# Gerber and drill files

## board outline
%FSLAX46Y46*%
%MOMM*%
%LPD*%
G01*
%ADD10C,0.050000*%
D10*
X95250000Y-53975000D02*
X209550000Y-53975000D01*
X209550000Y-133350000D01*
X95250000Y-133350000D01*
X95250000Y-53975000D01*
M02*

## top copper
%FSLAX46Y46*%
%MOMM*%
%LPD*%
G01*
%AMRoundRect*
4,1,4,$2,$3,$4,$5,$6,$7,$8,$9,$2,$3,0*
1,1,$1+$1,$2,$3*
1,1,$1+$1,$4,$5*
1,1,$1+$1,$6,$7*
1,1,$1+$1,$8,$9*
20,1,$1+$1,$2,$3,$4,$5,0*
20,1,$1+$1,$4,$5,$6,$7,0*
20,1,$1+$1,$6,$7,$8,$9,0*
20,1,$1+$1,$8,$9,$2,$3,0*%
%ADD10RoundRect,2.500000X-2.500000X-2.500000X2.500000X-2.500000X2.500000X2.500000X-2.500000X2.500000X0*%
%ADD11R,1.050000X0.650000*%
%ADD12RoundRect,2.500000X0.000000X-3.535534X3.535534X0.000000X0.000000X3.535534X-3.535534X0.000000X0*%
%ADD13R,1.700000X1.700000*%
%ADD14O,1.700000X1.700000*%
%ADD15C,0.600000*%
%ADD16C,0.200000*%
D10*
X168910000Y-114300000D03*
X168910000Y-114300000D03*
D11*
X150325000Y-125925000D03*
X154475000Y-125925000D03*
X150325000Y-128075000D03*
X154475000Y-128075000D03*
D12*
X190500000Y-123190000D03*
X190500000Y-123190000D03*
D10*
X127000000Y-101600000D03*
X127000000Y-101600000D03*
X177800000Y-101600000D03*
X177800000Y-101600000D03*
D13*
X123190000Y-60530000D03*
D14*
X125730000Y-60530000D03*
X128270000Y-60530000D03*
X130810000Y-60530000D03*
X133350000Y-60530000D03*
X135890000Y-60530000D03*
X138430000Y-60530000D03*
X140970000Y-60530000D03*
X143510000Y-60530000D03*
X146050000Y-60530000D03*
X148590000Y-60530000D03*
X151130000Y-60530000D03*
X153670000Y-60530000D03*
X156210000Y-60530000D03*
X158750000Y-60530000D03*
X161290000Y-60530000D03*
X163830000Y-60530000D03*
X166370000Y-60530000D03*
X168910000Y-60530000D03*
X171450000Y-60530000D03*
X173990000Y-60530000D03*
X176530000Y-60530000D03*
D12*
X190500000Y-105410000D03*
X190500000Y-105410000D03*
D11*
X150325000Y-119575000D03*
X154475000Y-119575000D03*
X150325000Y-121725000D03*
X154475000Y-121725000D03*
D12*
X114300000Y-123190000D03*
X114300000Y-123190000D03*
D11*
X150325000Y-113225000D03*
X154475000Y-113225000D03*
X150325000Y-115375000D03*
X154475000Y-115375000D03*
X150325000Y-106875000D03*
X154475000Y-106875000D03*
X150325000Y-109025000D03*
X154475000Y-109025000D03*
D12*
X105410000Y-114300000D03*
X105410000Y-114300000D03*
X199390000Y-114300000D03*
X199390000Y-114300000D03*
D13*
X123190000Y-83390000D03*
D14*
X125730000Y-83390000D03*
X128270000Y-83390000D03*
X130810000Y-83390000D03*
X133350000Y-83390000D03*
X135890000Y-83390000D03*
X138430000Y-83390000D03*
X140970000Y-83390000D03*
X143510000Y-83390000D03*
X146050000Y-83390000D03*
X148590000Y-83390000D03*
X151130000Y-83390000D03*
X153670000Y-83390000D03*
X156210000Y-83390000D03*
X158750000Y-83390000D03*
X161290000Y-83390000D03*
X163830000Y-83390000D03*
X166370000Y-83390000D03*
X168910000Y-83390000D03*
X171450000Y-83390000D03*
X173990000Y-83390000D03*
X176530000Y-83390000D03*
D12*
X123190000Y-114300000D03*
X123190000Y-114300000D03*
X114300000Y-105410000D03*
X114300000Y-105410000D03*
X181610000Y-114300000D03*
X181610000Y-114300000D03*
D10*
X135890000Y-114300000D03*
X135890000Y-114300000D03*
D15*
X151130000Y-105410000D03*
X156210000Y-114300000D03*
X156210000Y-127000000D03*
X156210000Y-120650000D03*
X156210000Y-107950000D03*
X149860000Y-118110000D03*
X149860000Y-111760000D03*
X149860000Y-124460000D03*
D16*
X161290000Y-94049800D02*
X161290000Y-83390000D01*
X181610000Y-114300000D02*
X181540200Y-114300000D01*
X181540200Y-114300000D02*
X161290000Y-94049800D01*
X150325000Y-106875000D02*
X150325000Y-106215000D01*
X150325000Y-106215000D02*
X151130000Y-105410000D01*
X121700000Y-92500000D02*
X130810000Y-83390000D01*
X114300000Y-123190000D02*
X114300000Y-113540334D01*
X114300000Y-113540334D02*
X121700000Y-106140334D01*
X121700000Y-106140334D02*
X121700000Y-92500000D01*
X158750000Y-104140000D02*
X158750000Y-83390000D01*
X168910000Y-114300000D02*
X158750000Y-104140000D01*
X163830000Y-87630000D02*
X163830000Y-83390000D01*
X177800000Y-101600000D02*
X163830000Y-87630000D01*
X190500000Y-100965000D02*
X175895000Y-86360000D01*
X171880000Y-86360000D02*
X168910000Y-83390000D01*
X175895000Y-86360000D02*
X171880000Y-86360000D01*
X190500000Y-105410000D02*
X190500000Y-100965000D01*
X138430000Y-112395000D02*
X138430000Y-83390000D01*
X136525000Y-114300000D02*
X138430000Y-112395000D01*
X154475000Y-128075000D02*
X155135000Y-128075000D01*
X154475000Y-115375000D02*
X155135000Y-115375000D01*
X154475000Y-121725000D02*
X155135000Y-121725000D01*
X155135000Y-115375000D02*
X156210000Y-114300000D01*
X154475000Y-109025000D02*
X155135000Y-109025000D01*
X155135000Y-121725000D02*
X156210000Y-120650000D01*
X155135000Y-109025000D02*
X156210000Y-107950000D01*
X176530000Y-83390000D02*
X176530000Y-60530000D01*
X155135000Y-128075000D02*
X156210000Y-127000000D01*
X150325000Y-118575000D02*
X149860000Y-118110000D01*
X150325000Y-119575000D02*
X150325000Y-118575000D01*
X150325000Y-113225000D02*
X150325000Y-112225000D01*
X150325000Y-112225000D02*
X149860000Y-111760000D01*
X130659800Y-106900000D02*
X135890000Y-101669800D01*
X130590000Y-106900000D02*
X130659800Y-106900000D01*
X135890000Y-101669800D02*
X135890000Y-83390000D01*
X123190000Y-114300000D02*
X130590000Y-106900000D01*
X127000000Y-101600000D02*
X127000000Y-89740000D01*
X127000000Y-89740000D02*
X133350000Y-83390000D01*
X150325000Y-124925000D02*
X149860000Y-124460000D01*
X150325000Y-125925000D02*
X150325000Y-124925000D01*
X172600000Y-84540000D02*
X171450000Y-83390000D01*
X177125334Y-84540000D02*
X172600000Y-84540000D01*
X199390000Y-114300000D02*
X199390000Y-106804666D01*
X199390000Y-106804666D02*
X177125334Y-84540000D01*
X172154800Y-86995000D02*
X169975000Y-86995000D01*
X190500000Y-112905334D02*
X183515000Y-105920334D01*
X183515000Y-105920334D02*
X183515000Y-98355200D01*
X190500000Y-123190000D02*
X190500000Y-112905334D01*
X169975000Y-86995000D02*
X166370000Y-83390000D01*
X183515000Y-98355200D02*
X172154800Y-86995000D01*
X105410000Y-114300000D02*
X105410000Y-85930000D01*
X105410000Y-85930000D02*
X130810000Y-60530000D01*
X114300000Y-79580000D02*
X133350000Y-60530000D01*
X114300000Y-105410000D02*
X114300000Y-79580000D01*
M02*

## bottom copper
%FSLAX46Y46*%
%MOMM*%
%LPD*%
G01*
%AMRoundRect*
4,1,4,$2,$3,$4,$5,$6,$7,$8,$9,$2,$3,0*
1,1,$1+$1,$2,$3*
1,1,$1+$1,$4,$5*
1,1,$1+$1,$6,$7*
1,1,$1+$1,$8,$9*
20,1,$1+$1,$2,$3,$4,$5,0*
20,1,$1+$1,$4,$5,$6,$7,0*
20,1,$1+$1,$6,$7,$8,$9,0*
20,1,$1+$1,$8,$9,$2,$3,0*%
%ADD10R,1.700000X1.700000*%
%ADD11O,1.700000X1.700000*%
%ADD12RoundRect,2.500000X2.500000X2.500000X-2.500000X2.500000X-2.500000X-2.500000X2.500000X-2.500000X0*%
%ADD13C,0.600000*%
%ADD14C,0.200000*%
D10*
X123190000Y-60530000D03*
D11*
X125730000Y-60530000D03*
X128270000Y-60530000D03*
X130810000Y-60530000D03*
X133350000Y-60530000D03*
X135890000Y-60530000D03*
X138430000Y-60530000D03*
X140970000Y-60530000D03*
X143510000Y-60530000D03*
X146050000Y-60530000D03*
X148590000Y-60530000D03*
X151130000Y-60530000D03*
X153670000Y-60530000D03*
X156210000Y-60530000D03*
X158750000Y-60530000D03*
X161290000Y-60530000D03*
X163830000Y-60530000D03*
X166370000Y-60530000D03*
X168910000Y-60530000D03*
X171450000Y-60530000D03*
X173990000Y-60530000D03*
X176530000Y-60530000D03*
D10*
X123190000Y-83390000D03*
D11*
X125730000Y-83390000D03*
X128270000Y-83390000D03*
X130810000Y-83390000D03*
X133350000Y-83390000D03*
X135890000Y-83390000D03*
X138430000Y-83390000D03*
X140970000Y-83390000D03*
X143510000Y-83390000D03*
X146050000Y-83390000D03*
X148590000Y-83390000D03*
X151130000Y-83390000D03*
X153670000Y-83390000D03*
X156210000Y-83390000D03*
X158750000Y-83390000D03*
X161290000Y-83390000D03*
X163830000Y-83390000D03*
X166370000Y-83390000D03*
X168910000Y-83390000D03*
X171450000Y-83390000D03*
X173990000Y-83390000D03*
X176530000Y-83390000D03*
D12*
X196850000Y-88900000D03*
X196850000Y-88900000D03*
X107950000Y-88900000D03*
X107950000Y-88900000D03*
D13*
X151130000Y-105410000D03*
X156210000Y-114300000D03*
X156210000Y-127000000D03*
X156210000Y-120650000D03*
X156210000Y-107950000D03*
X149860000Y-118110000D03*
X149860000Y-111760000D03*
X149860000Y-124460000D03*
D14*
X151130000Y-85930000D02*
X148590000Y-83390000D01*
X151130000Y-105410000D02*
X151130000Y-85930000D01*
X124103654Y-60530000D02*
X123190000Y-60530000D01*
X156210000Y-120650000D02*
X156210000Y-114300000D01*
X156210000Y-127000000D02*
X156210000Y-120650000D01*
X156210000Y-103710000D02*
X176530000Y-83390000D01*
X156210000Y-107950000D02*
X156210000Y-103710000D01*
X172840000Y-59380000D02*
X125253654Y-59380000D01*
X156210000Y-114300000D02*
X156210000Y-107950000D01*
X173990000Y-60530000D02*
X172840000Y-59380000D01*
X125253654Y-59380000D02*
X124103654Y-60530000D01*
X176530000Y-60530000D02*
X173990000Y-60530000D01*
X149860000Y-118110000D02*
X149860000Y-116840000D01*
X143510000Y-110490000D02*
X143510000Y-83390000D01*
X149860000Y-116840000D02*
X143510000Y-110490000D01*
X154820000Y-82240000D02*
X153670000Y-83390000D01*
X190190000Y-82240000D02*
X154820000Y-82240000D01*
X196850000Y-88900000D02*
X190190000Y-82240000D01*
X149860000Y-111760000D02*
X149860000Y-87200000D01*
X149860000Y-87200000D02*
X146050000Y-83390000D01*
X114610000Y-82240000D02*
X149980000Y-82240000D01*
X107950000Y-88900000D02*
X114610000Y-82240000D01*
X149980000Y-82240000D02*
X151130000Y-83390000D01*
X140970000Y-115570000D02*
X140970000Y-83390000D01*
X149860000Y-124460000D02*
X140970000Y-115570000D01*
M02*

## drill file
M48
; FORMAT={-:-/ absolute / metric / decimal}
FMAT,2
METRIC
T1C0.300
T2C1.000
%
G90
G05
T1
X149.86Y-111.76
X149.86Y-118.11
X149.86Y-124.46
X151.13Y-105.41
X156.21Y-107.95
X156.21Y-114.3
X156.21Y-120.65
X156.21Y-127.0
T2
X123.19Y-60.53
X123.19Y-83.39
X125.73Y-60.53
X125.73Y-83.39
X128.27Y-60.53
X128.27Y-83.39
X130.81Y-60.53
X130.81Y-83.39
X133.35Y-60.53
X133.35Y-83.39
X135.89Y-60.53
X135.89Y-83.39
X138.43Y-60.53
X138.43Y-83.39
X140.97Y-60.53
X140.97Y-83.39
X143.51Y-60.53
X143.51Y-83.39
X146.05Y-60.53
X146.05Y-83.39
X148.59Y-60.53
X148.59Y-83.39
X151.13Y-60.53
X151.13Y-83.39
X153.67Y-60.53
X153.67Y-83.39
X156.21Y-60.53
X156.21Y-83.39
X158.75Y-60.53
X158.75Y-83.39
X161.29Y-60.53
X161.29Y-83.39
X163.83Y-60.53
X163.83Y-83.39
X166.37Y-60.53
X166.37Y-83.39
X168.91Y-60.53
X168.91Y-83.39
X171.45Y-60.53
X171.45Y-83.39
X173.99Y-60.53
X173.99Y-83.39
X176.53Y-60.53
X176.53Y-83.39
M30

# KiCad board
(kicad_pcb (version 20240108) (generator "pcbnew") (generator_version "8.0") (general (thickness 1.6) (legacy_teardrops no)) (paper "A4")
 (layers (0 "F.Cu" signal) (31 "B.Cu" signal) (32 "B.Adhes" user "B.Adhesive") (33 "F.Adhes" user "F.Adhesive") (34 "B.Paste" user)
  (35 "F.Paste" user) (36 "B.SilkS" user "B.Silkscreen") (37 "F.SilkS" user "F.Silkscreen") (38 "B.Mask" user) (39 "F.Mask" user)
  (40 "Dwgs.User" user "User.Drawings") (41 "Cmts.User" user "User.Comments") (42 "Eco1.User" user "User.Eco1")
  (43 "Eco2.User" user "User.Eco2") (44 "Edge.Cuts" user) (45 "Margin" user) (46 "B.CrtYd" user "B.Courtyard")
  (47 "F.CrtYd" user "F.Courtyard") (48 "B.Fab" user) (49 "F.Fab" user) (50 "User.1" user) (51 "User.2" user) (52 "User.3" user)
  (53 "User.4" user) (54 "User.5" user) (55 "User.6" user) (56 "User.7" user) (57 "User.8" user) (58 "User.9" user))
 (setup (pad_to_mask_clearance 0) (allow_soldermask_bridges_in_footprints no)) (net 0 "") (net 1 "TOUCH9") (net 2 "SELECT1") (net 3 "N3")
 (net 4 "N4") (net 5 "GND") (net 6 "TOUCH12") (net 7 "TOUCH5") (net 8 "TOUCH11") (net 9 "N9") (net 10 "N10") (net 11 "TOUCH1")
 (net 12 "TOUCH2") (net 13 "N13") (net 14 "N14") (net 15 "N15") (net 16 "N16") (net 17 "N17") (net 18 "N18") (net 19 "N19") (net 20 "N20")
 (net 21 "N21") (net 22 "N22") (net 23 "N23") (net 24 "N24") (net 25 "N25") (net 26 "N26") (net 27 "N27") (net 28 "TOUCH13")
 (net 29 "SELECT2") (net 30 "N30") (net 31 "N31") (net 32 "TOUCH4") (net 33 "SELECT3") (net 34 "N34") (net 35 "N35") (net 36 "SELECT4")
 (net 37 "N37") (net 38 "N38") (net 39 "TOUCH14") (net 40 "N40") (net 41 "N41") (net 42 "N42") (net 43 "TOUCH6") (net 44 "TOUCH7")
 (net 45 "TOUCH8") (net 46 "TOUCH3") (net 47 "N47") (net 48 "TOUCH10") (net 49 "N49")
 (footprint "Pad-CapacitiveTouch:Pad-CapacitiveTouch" (layer "F.Cu") (at 168.91 114.3)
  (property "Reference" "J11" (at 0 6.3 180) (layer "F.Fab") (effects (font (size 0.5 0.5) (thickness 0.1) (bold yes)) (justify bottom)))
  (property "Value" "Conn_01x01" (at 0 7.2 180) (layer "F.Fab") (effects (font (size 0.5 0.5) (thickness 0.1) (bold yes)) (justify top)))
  (pad "1" smd roundrect (at 0 0) (size 10 10) (layers "F.Cu") (roundrect_rratio 0.25) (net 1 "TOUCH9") (thermal_bridge_angle 0))
  (pad "1" smd roundrect (at 0 0) (size 10 10) (layers "F.Cu" "F.Mask") (roundrect_rratio 0.25) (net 1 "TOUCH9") (thermal_bridge_angle 0)))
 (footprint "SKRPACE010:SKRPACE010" (layer "F.Cu") (at 152.4 127)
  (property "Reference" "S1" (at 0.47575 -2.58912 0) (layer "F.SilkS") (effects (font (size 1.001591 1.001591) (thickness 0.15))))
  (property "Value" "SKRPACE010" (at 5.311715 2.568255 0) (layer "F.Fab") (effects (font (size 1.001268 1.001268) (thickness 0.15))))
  (pad "1" smd rect (at -2.075 -1.075) (size 1.05 0.65) (layers "F.Cu" "F.Paste" "F.Mask") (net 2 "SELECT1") (solder_mask_margin 0.102))
  (pad "2" smd rect (at 2.075 -1.075) (size 1.05 0.65) (layers "F.Cu" "F.Paste" "F.Mask") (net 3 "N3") (solder_mask_margin 0.102))
  (pad "3" smd rect (at -2.075 1.075) (size 1.05 0.65) (layers "F.Cu" "F.Paste" "F.Mask") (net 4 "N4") (solder_mask_margin 0.102))
  (pad "4" smd rect (at 2.075 1.075) (size 1.05 0.65) (layers "F.Cu" "F.Paste" "F.Mask") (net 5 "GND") (solder_mask_margin 0.102)))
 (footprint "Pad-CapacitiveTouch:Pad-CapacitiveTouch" (layer "F.Cu") (at 190.5 123.19 45)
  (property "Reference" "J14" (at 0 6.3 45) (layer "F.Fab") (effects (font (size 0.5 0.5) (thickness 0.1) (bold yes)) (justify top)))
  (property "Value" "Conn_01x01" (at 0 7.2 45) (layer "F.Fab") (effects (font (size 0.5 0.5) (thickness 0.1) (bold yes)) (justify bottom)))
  (pad "1" smd roundrect (at 0 0 45) (size 10 10) (layers "F.Cu") (roundrect_rratio 0.25) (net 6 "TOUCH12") (thermal_bridge_angle 0))
  (pad "1" smd roundrect (at 0 0 45) (size 10 10) (layers "F.Cu" "F.Mask") (roundrect_rratio 0.25) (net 6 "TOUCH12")
   (thermal_bridge_angle 0)))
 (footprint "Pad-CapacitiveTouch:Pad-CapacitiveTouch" (layer "F.Cu") (at 127 101.6)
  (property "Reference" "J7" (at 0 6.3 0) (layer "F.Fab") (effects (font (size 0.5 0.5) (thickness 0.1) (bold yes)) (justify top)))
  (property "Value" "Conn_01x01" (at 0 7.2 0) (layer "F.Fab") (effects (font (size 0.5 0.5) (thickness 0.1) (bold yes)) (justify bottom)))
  (pad "1" smd roundrect (at 0 0) (size 10 10) (layers "F.Cu") (roundrect_rratio 0.25) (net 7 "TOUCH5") (thermal_bridge_angle 0))
  (pad "1" smd roundrect (at 0 0) (size 10 10) (layers "F.Cu" "F.Mask") (roundrect_rratio 0.25) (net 7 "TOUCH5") (thermal_bridge_angle 0)))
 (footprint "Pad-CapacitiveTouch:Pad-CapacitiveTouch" (layer "F.Cu") (at 177.8 101.6)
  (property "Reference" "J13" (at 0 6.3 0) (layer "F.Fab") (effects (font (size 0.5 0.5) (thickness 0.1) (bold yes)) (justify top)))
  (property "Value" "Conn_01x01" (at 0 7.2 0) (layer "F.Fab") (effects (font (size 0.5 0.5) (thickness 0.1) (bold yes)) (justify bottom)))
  (pad "1" smd roundrect (at 0 0) (size 10 10) (layers "F.Cu") (roundrect_rratio 0.25) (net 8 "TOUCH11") (thermal_bridge_angle 0))
  (pad "1" smd roundrect (at 0 0) (size 10 10) (layers "F.Cu" "F.Mask") (roundrect_rratio 0.25) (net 8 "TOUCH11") (thermal_bridge_angle 0)))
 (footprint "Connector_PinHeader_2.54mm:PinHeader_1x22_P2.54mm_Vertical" (layer "F.Cu") (at 123.19 60.53 90)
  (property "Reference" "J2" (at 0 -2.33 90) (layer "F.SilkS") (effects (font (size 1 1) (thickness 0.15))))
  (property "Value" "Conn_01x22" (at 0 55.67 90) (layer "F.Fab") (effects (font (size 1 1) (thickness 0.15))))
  (pad "1" thru_hole rect (at 0 0 90) (size 1.7 1.7) (drill 1) (layers "*.Cu" "*.Mask") (remove_unused_layers no) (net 5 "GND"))
  (pad "2" thru_hole oval (at 0 2.54 90) (size 1.7 1.7) (drill 1) (layers "*.Cu" "*.Mask") (remove_unused_layers no) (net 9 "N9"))
  (pad "3" thru_hole oval (at 0 5.08 90) (size 1.7 1.7) (drill 1) (layers "*.Cu" "*.Mask") (remove_unused_layers no) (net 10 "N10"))
  (pad "4" thru_hole oval (at 0 7.62 90) (size 1.7 1.7) (drill 1) (layers "*.Cu" "*.Mask") (remove_unused_layers no) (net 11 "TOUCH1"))
  (pad "5" thru_hole oval (at 0 10.16 90) (size 1.7 1.7) (drill 1) (layers "*.Cu" "*.Mask") (remove_unused_layers no) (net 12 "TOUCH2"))
  (pad "6" thru_hole oval (at 0 12.7 90) (size 1.7 1.7) (drill 1) (layers "*.Cu" "*.Mask") (remove_unused_layers no) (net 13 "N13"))
  (pad "7" thru_hole oval (at 0 15.24 90) (size 1.7 1.7) (drill 1) (layers "*.Cu" "*.Mask") (remove_unused_layers no) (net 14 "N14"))
  (pad "8" thru_hole oval (at 0 17.78 90) (size 1.7 1.7) (drill 1) (layers "*.Cu" "*.Mask") (remove_unused_layers no) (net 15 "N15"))
  (pad "9" thru_hole oval (at 0 20.32 90) (size 1.7 1.7) (drill 1) (layers "*.Cu" "*.Mask") (remove_unused_layers no) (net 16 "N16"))
  (pad "10" thru_hole oval (at 0 22.86 90) (size 1.7 1.7) (drill 1) (layers "*.Cu" "*.Mask") (remove_unused_layers no) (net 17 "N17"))
  (pad "11" thru_hole oval (at 0 25.4 90) (size 1.7 1.7) (drill 1) (layers "*.Cu" "*.Mask") (remove_unused_layers no) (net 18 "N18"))
  (pad "12" thru_hole oval (at 0 27.94 90) (size 1.7 1.7) (drill 1) (layers "*.Cu" "*.Mask") (remove_unused_layers no) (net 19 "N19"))
  (pad "13" thru_hole oval (at 0 30.48 90) (size 1.7 1.7) (drill 1) (layers "*.Cu" "*.Mask") (remove_unused_layers no) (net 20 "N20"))
  (pad "14" thru_hole oval (at 0 33.02 90) (size 1.7 1.7) (drill 1) (layers "*.Cu" "*.Mask") (remove_unused_layers no) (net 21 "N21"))
  (pad "15" thru_hole oval (at 0 35.56 90) (size 1.7 1.7) (drill 1) (layers "*.Cu" "*.Mask") (remove_unused_layers no) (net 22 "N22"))
  (pad "16" thru_hole oval (at 0 38.1 90) (size 1.7 1.7) (drill 1) (layers "*.Cu" "*.Mask") (remove_unused_layers no) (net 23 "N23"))
  (pad "17" thru_hole oval (at 0 40.64 90) (size 1.7 1.7) (drill 1) (layers "*.Cu" "*.Mask") (remove_unused_layers no) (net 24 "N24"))
  (pad "18" thru_hole oval (at 0 43.18 90) (size 1.7 1.7) (drill 1) (layers "*.Cu" "*.Mask") (remove_unused_layers no) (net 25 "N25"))
  (pad "19" thru_hole oval (at 0 45.72 90) (size 1.7 1.7) (drill 1) (layers "*.Cu" "*.Mask") (remove_unused_layers no) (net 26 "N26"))
  (pad "20" thru_hole oval (at 0 48.26 90) (size 1.7 1.7) (drill 1) (layers "*.Cu" "*.Mask") (remove_unused_layers no) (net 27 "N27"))
  (pad "21" thru_hole oval (at 0 50.8 90) (size 1.7 1.7) (drill 1) (layers "*.Cu" "*.Mask") (remove_unused_layers no) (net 5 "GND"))
  (pad "22" thru_hole oval (at 0 53.34 90) (size 1.7 1.7) (drill 1) (layers "*.Cu" "*.Mask") (remove_unused_layers no) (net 5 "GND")))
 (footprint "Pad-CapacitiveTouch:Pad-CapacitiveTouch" (layer "F.Cu") (at 190.5 105.41 45)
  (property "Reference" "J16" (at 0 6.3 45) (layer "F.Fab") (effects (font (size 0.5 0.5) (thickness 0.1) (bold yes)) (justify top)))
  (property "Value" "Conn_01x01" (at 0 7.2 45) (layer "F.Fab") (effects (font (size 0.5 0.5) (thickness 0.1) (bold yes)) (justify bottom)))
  (pad "1" smd roundrect (at 0 0 45) (size 10 10) (layers "F.Cu") (roundrect_rratio 0.25) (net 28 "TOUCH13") (thermal_bridge_angle 0))
  (pad "1" smd roundrect (at 0 0 45) (size 10 10) (layers "F.Cu" "F.Mask") (roundrect_rratio 0.25) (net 28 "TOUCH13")
   (thermal_bridge_angle 0)))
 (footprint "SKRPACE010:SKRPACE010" (layer "F.Cu") (at 152.4 120.65)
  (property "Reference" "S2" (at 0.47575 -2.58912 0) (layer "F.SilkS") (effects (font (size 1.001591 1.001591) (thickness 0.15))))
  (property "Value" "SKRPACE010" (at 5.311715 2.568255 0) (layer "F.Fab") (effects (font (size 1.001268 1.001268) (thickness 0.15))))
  (pad "1" smd rect (at -2.075 -1.075) (size 1.05 0.65) (layers "F.Cu" "F.Paste" "F.Mask") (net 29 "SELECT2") (solder_mask_margin 0.102))
  (pad "2" smd rect (at 2.075 -1.075) (size 1.05 0.65) (layers "F.Cu" "F.Paste" "F.Mask") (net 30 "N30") (solder_mask_margin 0.102))
  (pad "3" smd rect (at -2.075 1.075) (size 1.05 0.65) (layers "F.Cu" "F.Paste" "F.Mask") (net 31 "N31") (solder_mask_margin 0.102))
  (pad "4" smd rect (at 2.075 1.075) (size 1.05 0.65) (layers "F.Cu" "F.Paste" "F.Mask") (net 5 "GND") (solder_mask_margin 0.102)))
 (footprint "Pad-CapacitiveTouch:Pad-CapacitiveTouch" (layer "F.Cu") (at 114.3 123.19 45)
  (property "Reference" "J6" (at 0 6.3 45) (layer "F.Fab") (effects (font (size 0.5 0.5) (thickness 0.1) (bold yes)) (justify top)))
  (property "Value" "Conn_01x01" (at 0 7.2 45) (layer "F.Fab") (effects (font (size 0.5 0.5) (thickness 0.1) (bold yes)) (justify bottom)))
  (pad "1" smd roundrect (at 0 0 45) (size 10 10) (layers "F.Cu") (roundrect_rratio 0.25) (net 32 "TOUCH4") (thermal_bridge_angle 0))
  (pad "1" smd roundrect (at 0 0 45) (size 10 10) (layers "F.Cu" "F.Mask") (roundrect_rratio 0.25) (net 32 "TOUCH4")
   (thermal_bridge_angle 0)))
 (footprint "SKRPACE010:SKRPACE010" (layer "F.Cu") (at 152.4 114.3)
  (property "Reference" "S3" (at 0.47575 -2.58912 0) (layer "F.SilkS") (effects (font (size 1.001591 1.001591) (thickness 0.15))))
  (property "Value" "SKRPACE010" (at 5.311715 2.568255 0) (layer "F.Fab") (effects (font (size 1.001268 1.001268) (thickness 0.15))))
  (pad "1" smd rect (at -2.075 -1.075) (size 1.05 0.65) (layers "F.Cu" "F.Paste" "F.Mask") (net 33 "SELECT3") (solder_mask_margin 0.102))
  (pad "2" smd rect (at 2.075 -1.075) (size 1.05 0.65) (layers "F.Cu" "F.Paste" "F.Mask") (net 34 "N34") (solder_mask_margin 0.102))
  (pad "3" smd rect (at -2.075 1.075) (size 1.05 0.65) (layers "F.Cu" "F.Paste" "F.Mask") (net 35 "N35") (solder_mask_margin 0.102))
  (pad "4" smd rect (at 2.075 1.075) (size 1.05 0.65) (layers "F.Cu" "F.Paste" "F.Mask") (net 5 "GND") (solder_mask_margin 0.102)))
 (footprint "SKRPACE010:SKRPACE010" (layer "F.Cu") (at 152.4 107.95)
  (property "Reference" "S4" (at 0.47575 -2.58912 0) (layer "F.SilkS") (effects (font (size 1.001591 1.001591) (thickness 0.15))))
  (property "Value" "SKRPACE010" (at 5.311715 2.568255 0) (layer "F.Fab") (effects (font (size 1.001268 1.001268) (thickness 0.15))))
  (pad "1" smd rect (at -2.075 -1.075) (size 1.05 0.65) (layers "F.Cu" "F.Paste" "F.Mask") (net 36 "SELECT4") (solder_mask_margin 0.102))
  (pad "2" smd rect (at 2.075 -1.075) (size 1.05 0.65) (layers "F.Cu" "F.Paste" "F.Mask") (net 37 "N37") (solder_mask_margin 0.102))
  (pad "3" smd rect (at -2.075 1.075) (size 1.05 0.65) (layers "F.Cu" "F.Paste" "F.Mask") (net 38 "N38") (solder_mask_margin 0.102))
  (pad "4" smd rect (at 2.075 1.075) (size 1.05 0.65) (layers "F.Cu" "F.Paste" "F.Mask") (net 5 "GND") (solder_mask_margin 0.102)))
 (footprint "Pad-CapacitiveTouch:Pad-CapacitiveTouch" (layer "F.Cu") (at 105.41 114.3 45)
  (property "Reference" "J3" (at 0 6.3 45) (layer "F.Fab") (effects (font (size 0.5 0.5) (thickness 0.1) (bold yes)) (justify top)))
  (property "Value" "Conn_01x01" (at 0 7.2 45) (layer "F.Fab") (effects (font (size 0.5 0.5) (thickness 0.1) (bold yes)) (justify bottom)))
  (pad "1" smd roundrect (at 0 0 45) (size 10 10) (layers "F.Cu") (roundrect_rratio 0.25) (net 11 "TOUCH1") (thermal_bridge_angle 0))
  (pad "1" smd roundrect (at 0 0 45) (size 10 10) (layers "F.Cu" "F.Mask") (roundrect_rratio 0.25) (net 11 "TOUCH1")
   (thermal_bridge_angle 0)))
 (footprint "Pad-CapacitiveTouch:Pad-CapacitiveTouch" (layer "F.Cu") (at 199.39 114.3 45)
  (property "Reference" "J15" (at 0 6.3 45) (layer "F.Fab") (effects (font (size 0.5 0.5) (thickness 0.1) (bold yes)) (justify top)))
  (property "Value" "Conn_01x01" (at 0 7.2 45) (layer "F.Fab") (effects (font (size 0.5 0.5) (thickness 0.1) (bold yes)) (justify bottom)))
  (pad "1" smd roundrect (at 0 0 45) (size 10 10) (layers "F.Cu") (roundrect_rratio 0.25) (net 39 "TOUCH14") (thermal_bridge_angle 0))
  (pad "1" smd roundrect (at 0 0 45) (size 10 10) (layers "F.Cu" "F.Mask") (roundrect_rratio 0.25) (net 39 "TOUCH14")
   (thermal_bridge_angle 0)))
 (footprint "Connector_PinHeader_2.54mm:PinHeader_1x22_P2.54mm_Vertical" (layer "F.Cu") (at 123.19 83.39 90)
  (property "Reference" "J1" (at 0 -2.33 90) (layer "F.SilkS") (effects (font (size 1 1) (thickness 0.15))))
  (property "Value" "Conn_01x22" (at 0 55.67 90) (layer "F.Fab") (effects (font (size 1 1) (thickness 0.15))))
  (pad "1" thru_hole rect (at 0 0 90) (size 1.7 1.7) (drill 1) (layers "*.Cu" "*.Mask") (remove_unused_layers no) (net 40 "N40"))
  (pad "2" thru_hole oval (at 0 2.54 90) (size 1.7 1.7) (drill 1) (layers "*.Cu" "*.Mask") (remove_unused_layers no) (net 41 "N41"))
  (pad "3" thru_hole oval (at 0 5.08 90) (size 1.7 1.7) (drill 1) (layers "*.Cu" "*.Mask") (remove_unused_layers no) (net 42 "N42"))
  (pad "4" thru_hole oval (at 0 7.62 90) (size 1.7 1.7) (drill 1) (layers "*.Cu" "*.Mask") (remove_unused_layers no) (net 32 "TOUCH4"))
  (pad "5" thru_hole oval (at 0 10.16 90) (size 1.7 1.7) (drill 1) (layers "*.Cu" "*.Mask") (remove_unused_layers no) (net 7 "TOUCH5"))
  (pad "6" thru_hole oval (at 0 12.7 90) (size 1.7 1.7) (drill 1) (layers "*.Cu" "*.Mask") (remove_unused_layers no) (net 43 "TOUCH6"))
  (pad "7" thru_hole oval (at 0 15.24 90) (size 1.7 1.7) (drill 1) (layers "*.Cu" "*.Mask") (remove_unused_layers no) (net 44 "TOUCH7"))
  (pad "8" thru_hole oval (at 0 17.78 90) (size 1.7 1.7) (drill 1) (layers "*.Cu" "*.Mask") (remove_unused_layers no) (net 2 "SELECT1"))
  (pad "9" thru_hole oval (at 0 20.32 90) (size 1.7 1.7) (drill 1) (layers "*.Cu" "*.Mask") (remove_unused_layers no) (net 29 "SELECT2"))
  (pad "10" thru_hole oval (at 0 22.86 90) (size 1.7 1.7) (drill 1) (layers "*.Cu" "*.Mask") (remove_unused_layers no) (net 33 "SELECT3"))
  (pad "11" thru_hole oval (at 0 25.4 90) (size 1.7 1.7) (drill 1) (layers "*.Cu" "*.Mask") (remove_unused_layers no) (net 36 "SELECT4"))
  (pad "12" thru_hole oval (at 0 27.94 90) (size 1.7 1.7) (drill 1) (layers "*.Cu" "*.Mask") (remove_unused_layers no) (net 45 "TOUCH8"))
  (pad "13" thru_hole oval (at 0 30.48 90) (size 1.7 1.7) (drill 1) (layers "*.Cu" "*.Mask") (remove_unused_layers no) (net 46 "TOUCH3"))
  (pad "14" thru_hole oval (at 0 33.02 90) (size 1.7 1.7) (drill 1) (layers "*.Cu" "*.Mask") (remove_unused_layers no) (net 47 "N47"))
  (pad "15" thru_hole oval (at 0 35.56 90) (size 1.7 1.7) (drill 1) (layers "*.Cu" "*.Mask") (remove_unused_layers no) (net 1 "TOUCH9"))
  (pad "16" thru_hole oval (at 0 38.1 90) (size 1.7 1.7) (drill 1) (layers "*.Cu" "*.Mask") (remove_unused_layers no) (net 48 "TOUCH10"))
  (pad "17" thru_hole oval (at 0 40.64 90) (size 1.7 1.7) (drill 1) (layers "*.Cu" "*.Mask") (remove_unused_layers no) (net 8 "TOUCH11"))
  (pad "18" thru_hole oval (at 0 43.18 90) (size 1.7 1.7) (drill 1) (layers "*.Cu" "*.Mask") (remove_unused_layers no) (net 6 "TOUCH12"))
  (pad "19" thru_hole oval (at 0 45.72 90) (size 1.7 1.7) (drill 1) (layers "*.Cu" "*.Mask") (remove_unused_layers no) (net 28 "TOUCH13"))
  (pad "20" thru_hole oval (at 0 48.26 90) (size 1.7 1.7) (drill 1) (layers "*.Cu" "*.Mask") (remove_unused_layers no) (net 39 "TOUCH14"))
  (pad "21" thru_hole oval (at 0 50.8 90) (size 1.7 1.7) (drill 1) (layers "*.Cu" "*.Mask") (remove_unused_layers no) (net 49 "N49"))
  (pad "22" thru_hole oval (at 0 53.34 90) (size 1.7 1.7) (drill 1) (layers "*.Cu" "*.Mask") (remove_unused_layers no) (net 5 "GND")))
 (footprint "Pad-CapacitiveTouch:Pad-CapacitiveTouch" (layer "F.Cu") (at 123.19 114.3 45)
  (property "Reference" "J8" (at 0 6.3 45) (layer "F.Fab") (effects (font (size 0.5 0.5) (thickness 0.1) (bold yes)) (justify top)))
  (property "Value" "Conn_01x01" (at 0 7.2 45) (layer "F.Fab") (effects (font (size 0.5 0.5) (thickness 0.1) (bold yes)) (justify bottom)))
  (pad "1" smd roundrect (at 0 0 45) (size 10 10) (layers "F.Cu") (roundrect_rratio 0.25) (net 43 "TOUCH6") (thermal_bridge_angle 0))
  (pad "1" smd roundrect (at 0 0 45) (size 10 10) (layers "F.Cu" "F.Mask") (roundrect_rratio 0.25) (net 43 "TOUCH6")
   (thermal_bridge_angle 0)))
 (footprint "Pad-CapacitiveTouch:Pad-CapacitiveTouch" (layer "F.Cu") (at 114.3 105.41 45)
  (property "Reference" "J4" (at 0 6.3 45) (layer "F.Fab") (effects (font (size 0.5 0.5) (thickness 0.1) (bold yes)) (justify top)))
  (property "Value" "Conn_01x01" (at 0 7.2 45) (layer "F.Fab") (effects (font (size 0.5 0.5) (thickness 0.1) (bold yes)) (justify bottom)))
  (pad "1" smd roundrect (at 0 0 45) (size 10 10) (layers "F.Cu") (roundrect_rratio 0.25) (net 12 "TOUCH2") (thermal_bridge_angle 0))
  (pad "1" smd roundrect (at 0 0 45) (size 10 10) (layers "F.Cu" "F.Mask") (roundrect_rratio 0.25) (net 12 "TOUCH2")
   (thermal_bridge_angle 0)))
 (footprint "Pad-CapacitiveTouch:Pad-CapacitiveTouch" (layer "F.Cu") (at 181.61 114.3 45)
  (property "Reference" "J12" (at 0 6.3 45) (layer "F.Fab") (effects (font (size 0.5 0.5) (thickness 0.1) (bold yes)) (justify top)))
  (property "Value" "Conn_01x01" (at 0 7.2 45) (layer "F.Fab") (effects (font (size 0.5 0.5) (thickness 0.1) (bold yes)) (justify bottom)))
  (pad "1" smd roundrect (at 0 0 45) (size 10 10) (layers "F.Cu") (roundrect_rratio 0.25) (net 48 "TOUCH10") (thermal_bridge_angle 0))
  (pad "1" smd roundrect (at 0 0 45) (size 10 10) (layers "F.Cu" "F.Mask") (roundrect_rratio 0.25) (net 48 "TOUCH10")
   (thermal_bridge_angle 0)))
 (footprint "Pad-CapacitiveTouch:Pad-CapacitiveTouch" (layer "F.Cu") (at 135.89 114.3)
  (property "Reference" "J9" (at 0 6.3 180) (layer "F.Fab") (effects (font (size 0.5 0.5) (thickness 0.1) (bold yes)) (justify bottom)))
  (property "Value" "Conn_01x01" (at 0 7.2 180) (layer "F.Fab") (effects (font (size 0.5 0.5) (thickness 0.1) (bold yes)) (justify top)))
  (pad "1" smd roundrect (at 0 0) (size 10 10) (layers "F.Cu") (roundrect_rratio 0.25) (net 44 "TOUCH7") (thermal_bridge_angle 0))
  (pad "1" smd roundrect (at 0 0) (size 10 10) (layers "F.Cu" "F.Mask") (roundrect_rratio 0.25) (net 44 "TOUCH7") (thermal_bridge_angle 0)))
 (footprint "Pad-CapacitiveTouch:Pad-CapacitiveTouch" (layer "B.Cu") (at 196.85 88.9 180)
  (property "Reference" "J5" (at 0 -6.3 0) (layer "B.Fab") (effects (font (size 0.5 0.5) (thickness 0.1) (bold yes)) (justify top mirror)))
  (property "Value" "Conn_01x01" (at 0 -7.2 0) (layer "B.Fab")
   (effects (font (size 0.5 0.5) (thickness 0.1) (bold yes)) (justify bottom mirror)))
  (pad "1" smd roundrect (at 0 0 180) (size 10 10) (layers "B.Cu") (roundrect_rratio 0.25) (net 46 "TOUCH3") (thermal_bridge_angle 0))
  (pad "1" smd roundrect (at 0 0 180) (size 10 10) (layers "B.Cu" "B.Mask") (roundrect_rratio 0.25) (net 46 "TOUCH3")
   (thermal_bridge_angle 0)))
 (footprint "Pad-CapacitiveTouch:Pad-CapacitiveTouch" (layer "B.Cu") (at 107.95 88.9 180)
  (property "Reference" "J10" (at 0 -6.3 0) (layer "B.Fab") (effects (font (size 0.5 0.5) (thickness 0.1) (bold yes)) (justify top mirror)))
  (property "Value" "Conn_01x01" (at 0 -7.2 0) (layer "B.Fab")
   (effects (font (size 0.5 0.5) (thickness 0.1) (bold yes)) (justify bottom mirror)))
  (pad "1" smd roundrect (at 0 0 180) (size 10 10) (layers "B.Cu") (roundrect_rratio 0.25) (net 45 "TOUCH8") (thermal_bridge_angle 0))
  (pad "1" smd roundrect (at 0 0 180) (size 10 10) (layers "B.Cu" "B.Mask") (roundrect_rratio 0.25) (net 45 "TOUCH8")
   (thermal_bridge_angle 0)))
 (gr_rect (start 95.25 53.975) (end 209.55 133.35) (stroke (width 0.05) (type default)) (fill none) (layer "Edge.Cuts"))
 (segment (start 161.29 94.0498) (end 161.29 83.39) (width 0.2) (layer "F.Cu") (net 48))
 (segment (start 181.61 114.3) (end 181.5402 114.3) (width 0.2) (layer "F.Cu") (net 48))
 (segment (start 181.5402 114.3) (end 161.29 94.0498) (width 0.2) (layer "F.Cu") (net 48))
 (segment (start 150.325 106.875) (end 150.325 106.215) (width 0.2) (layer "F.Cu") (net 36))
 (segment (start 150.325 106.215) (end 151.13 105.41) (width 0.2) (layer "F.Cu") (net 36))
 (via (at 151.13 105.41) (size 0.6) (drill 0.3) (layers "F.Cu" "B.Cu") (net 36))
 (segment (start 151.13 85.93) (end 148.59 83.39) (width 0.2) (layer "B.Cu") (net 36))
 (segment (start 151.13 105.41) (end 151.13 85.93) (width 0.2) (layer "B.Cu") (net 36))
 (segment (start 121.7 92.5) (end 130.81 83.39) (width 0.2) (layer "F.Cu") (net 32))
 (segment (start 114.3 123.19) (end 114.3 113.540334) (width 0.2) (layer "F.Cu") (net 32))
 (segment (start 114.3 113.540334) (end 121.7 106.140334) (width 0.2) (layer "F.Cu") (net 32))
 (segment (start 121.7 106.140334) (end 121.7 92.5) (width 0.2) (layer "F.Cu") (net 32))
 (segment (start 158.75 104.14) (end 158.75 83.39) (width 0.2) (layer "F.Cu") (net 1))
 (segment (start 168.91 114.3) (end 158.75 104.14) (width 0.2) (layer "F.Cu") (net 1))
 (segment (start 163.83 87.63) (end 163.83 83.39) (width 0.2) (layer "F.Cu") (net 8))
 (segment (start 177.8 101.6) (end 163.83 87.63) (width 0.2) (layer "F.Cu") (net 8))
 (segment (start 190.5 100.965) (end 175.895 86.36) (width 0.2) (layer "F.Cu") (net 28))
 (segment (start 171.88 86.36) (end 168.91 83.39) (width 0.2) (layer "F.Cu") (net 28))
 (segment (start 175.895 86.36) (end 171.88 86.36) (width 0.2) (layer "F.Cu") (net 28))
 (segment (start 190.5 105.41) (end 190.5 100.965) (width 0.2) (layer "F.Cu") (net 28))
 (segment (start 138.43 112.395) (end 138.43 83.39) (width 0.2) (layer "F.Cu") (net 44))
 (segment (start 136.525 114.3) (end 138.43 112.395) (width 0.2) (layer "F.Cu") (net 44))
 (segment (start 154.475 128.075) (end 155.135 128.075) (width 0.2) (layer "F.Cu") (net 5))
 (segment (start 154.475 115.375) (end 155.135 115.375) (width 0.2) (layer "F.Cu") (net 5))
 (segment (start 154.475 121.725) (end 155.135 121.725) (width 0.2) (layer "F.Cu") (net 5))
 (segment (start 155.135 115.375) (end 156.21 114.3) (width 0.2) (layer "F.Cu") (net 5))
 (segment (start 154.475 109.025) (end 155.135 109.025) (width 0.2) (layer "F.Cu") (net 5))
 (segment (start 155.135 121.725) (end 156.21 120.65) (width 0.2) (layer "F.Cu") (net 5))
 (segment (start 155.135 109.025) (end 156.21 107.95) (width 0.2) (layer "F.Cu") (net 5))
 (segment (start 176.53 83.39) (end 176.53 60.53) (width 0.2) (layer "F.Cu") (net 5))
 (segment (start 155.135 128.075) (end 156.21 127) (width 0.2) (layer "F.Cu") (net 5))
 (via (at 156.21 114.3) (size 0.6) (drill 0.3) (layers "F.Cu" "B.Cu") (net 5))
 (via (at 156.21 127) (size 0.6) (drill 0.3) (layers "F.Cu" "B.Cu") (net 5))
 (via (at 156.21 120.65) (size 0.6) (drill 0.3) (layers "F.Cu" "B.Cu") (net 5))
 (via (at 156.21 107.95) (size 0.6) (drill 0.3) (layers "F.Cu" "B.Cu") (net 5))
 (segment (start 124.103654 60.53) (end 123.19 60.53) (width 0.2) (layer "B.Cu") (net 5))
 (segment (start 156.21 120.65) (end 156.21 114.3) (width 0.2) (layer "B.Cu") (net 5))
 (segment (start 156.21 127) (end 156.21 120.65) (width 0.2) (layer "B.Cu") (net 5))
 (segment (start 156.21 103.71) (end 176.53 83.39) (width 0.2) (layer "B.Cu") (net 5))
 (segment (start 156.21 107.95) (end 156.21 103.71) (width 0.2) (layer "B.Cu") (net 5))
 (segment (start 172.84 59.38) (end 125.253654 59.38) (width 0.2) (layer "B.Cu") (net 5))
 (segment (start 156.21 114.3) (end 156.21 107.95) (width 0.2) (layer "B.Cu") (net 5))
 (segment (start 173.99 60.53) (end 172.84 59.38) (width 0.2) (layer "B.Cu") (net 5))
 (segment (start 125.253654 59.38) (end 124.103654 60.53) (width 0.2) (layer "B.Cu") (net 5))
 (segment (start 176.53 60.53) (end 173.99 60.53) (width 0.2) (layer "B.Cu") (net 5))
 (segment (start 150.325 118.575) (end 149.86 118.11) (width 0.2) (layer "F.Cu") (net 29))
 (segment (start 150.325 119.575) (end 150.325 118.575) (width 0.2) (layer "F.Cu") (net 29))
 (via (at 149.86 118.11) (size 0.6) (drill 0.3) (layers "F.Cu" "B.Cu") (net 29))
 (segment (start 149.86 118.11) (end 149.86 116.84) (width 0.2) (layer "B.Cu") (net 29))
 (segment (start 143.51 110.49) (end 143.51 83.39) (width 0.2) (layer "B.Cu") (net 29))
 (segment (start 149.86 116.84) (end 143.51 110.49) (width 0.2) (layer "B.Cu") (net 29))
 (segment (start 154.82 82.24) (end 153.67 83.39) (width 0.2) (layer "B.Cu") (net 46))
 (segment (start 190.19 82.24) (end 154.82 82.24) (width 0.2) (layer "B.Cu") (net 46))
 (segment (start 196.85 88.9) (end 190.19 82.24) (width 0.2) (layer "B.Cu") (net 46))
 (segment (start 150.325 113.225) (end 150.325 112.225) (width 0.2) (layer "F.Cu") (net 33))
 (segment (start 150.325 112.225) (end 149.86 111.76) (width 0.2) (layer "F.Cu") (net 33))
 (via (at 149.86 111.76) (size 0.6) (drill 0.3) (layers "F.Cu" "B.Cu") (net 33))
 (segment (start 149.86 111.76) (end 149.86 87.2) (width 0.2) (layer "B.Cu") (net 33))
 (segment (start 149.86 87.2) (end 146.05 83.39) (width 0.2) (layer "B.Cu") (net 33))
 (segment (start 130.6598 106.9) (end 135.89 101.6698) (width 0.2) (layer "F.Cu") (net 43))
 (segment (start 130.59 106.9) (end 130.6598 106.9) (width 0.2) (layer "F.Cu") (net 43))
 (segment (start 135.89 101.6698) (end 135.89 83.39) (width 0.2) (layer "F.Cu") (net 43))
 (segment (start 123.19 114.3) (end 130.59 106.9) (width 0.2) (layer "F.Cu") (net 43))
 (segment (start 114.61 82.24) (end 149.98 82.24) (width 0.2) (layer "B.Cu") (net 45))
 (segment (start 107.95 88.9) (end 114.61 82.24) (width 0.2) (layer "B.Cu") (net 45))
 (segment (start 149.98 82.24) (end 151.13 83.39) (width 0.2) (layer "B.Cu") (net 45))
 (segment (start 127 101.6) (end 127 89.74) (width 0.2) (layer "F.Cu") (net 7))
 (segment (start 127 89.74) (end 133.35 83.39) (width 0.2) (layer "F.Cu") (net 7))
 (segment (start 150.325 124.925) (end 149.86 124.46) (width 0.2) (layer "F.Cu") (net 2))
 (segment (start 150.325 125.925) (end 150.325 124.925) (width 0.2) (layer "F.Cu") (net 2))
 (via (at 149.86 124.46) (size 0.6) (drill 0.3) (layers "F.Cu" "B.Cu") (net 2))
 (segment (start 140.97 115.57) (end 140.97 83.39) (width 0.2) (layer "B.Cu") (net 2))
 (segment (start 149.86 124.46) (end 140.97 115.57) (width 0.2) (layer "B.Cu") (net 2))
 (segment (start 172.6 84.54) (end 171.45 83.39) (width 0.2) (layer "F.Cu") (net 39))
 (segment (start 177.125334 84.54) (end 172.6 84.54) (width 0.2) (layer "F.Cu") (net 39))
 (segment (start 199.39 114.3) (end 199.39 106.804666) (width 0.2) (layer "F.Cu") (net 39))
 (segment (start 199.39 106.804666) (end 177.125334 84.54) (width 0.2) (layer "F.Cu") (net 39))
 (segment (start 172.1548 86.995) (end 169.975 86.995) (width 0.2) (layer "F.Cu") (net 6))
 (segment (start 190.5 112.905334) (end 183.515 105.920334) (width 0.2) (layer "F.Cu") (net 6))
 (segment (start 183.515 105.920334) (end 183.515 98.3552) (width 0.2) (layer "F.Cu") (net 6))
 (segment (start 190.5 123.19) (end 190.5 112.905334) (width 0.2) (layer "F.Cu") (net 6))
 (segment (start 169.975 86.995) (end 166.37 83.39) (width 0.2) (layer "F.Cu") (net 6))
 (segment (start 183.515 98.3552) (end 172.1548 86.995) (width 0.2) (layer "F.Cu") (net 6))
 (segment (start 105.41 114.3) (end 105.41 85.93) (width 0.2) (layer "F.Cu") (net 11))
 (segment (start 105.41 85.93) (end 130.81 60.53) (width 0.2) (layer "F.Cu") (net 11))
 (segment (start 114.3 79.58) (end 133.35 60.53) (width 0.2) (layer "F.Cu") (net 12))
 (segment (start 114.3 105.41) (end 114.3 79.58) (width 0.2) (layer "F.Cu") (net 12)))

